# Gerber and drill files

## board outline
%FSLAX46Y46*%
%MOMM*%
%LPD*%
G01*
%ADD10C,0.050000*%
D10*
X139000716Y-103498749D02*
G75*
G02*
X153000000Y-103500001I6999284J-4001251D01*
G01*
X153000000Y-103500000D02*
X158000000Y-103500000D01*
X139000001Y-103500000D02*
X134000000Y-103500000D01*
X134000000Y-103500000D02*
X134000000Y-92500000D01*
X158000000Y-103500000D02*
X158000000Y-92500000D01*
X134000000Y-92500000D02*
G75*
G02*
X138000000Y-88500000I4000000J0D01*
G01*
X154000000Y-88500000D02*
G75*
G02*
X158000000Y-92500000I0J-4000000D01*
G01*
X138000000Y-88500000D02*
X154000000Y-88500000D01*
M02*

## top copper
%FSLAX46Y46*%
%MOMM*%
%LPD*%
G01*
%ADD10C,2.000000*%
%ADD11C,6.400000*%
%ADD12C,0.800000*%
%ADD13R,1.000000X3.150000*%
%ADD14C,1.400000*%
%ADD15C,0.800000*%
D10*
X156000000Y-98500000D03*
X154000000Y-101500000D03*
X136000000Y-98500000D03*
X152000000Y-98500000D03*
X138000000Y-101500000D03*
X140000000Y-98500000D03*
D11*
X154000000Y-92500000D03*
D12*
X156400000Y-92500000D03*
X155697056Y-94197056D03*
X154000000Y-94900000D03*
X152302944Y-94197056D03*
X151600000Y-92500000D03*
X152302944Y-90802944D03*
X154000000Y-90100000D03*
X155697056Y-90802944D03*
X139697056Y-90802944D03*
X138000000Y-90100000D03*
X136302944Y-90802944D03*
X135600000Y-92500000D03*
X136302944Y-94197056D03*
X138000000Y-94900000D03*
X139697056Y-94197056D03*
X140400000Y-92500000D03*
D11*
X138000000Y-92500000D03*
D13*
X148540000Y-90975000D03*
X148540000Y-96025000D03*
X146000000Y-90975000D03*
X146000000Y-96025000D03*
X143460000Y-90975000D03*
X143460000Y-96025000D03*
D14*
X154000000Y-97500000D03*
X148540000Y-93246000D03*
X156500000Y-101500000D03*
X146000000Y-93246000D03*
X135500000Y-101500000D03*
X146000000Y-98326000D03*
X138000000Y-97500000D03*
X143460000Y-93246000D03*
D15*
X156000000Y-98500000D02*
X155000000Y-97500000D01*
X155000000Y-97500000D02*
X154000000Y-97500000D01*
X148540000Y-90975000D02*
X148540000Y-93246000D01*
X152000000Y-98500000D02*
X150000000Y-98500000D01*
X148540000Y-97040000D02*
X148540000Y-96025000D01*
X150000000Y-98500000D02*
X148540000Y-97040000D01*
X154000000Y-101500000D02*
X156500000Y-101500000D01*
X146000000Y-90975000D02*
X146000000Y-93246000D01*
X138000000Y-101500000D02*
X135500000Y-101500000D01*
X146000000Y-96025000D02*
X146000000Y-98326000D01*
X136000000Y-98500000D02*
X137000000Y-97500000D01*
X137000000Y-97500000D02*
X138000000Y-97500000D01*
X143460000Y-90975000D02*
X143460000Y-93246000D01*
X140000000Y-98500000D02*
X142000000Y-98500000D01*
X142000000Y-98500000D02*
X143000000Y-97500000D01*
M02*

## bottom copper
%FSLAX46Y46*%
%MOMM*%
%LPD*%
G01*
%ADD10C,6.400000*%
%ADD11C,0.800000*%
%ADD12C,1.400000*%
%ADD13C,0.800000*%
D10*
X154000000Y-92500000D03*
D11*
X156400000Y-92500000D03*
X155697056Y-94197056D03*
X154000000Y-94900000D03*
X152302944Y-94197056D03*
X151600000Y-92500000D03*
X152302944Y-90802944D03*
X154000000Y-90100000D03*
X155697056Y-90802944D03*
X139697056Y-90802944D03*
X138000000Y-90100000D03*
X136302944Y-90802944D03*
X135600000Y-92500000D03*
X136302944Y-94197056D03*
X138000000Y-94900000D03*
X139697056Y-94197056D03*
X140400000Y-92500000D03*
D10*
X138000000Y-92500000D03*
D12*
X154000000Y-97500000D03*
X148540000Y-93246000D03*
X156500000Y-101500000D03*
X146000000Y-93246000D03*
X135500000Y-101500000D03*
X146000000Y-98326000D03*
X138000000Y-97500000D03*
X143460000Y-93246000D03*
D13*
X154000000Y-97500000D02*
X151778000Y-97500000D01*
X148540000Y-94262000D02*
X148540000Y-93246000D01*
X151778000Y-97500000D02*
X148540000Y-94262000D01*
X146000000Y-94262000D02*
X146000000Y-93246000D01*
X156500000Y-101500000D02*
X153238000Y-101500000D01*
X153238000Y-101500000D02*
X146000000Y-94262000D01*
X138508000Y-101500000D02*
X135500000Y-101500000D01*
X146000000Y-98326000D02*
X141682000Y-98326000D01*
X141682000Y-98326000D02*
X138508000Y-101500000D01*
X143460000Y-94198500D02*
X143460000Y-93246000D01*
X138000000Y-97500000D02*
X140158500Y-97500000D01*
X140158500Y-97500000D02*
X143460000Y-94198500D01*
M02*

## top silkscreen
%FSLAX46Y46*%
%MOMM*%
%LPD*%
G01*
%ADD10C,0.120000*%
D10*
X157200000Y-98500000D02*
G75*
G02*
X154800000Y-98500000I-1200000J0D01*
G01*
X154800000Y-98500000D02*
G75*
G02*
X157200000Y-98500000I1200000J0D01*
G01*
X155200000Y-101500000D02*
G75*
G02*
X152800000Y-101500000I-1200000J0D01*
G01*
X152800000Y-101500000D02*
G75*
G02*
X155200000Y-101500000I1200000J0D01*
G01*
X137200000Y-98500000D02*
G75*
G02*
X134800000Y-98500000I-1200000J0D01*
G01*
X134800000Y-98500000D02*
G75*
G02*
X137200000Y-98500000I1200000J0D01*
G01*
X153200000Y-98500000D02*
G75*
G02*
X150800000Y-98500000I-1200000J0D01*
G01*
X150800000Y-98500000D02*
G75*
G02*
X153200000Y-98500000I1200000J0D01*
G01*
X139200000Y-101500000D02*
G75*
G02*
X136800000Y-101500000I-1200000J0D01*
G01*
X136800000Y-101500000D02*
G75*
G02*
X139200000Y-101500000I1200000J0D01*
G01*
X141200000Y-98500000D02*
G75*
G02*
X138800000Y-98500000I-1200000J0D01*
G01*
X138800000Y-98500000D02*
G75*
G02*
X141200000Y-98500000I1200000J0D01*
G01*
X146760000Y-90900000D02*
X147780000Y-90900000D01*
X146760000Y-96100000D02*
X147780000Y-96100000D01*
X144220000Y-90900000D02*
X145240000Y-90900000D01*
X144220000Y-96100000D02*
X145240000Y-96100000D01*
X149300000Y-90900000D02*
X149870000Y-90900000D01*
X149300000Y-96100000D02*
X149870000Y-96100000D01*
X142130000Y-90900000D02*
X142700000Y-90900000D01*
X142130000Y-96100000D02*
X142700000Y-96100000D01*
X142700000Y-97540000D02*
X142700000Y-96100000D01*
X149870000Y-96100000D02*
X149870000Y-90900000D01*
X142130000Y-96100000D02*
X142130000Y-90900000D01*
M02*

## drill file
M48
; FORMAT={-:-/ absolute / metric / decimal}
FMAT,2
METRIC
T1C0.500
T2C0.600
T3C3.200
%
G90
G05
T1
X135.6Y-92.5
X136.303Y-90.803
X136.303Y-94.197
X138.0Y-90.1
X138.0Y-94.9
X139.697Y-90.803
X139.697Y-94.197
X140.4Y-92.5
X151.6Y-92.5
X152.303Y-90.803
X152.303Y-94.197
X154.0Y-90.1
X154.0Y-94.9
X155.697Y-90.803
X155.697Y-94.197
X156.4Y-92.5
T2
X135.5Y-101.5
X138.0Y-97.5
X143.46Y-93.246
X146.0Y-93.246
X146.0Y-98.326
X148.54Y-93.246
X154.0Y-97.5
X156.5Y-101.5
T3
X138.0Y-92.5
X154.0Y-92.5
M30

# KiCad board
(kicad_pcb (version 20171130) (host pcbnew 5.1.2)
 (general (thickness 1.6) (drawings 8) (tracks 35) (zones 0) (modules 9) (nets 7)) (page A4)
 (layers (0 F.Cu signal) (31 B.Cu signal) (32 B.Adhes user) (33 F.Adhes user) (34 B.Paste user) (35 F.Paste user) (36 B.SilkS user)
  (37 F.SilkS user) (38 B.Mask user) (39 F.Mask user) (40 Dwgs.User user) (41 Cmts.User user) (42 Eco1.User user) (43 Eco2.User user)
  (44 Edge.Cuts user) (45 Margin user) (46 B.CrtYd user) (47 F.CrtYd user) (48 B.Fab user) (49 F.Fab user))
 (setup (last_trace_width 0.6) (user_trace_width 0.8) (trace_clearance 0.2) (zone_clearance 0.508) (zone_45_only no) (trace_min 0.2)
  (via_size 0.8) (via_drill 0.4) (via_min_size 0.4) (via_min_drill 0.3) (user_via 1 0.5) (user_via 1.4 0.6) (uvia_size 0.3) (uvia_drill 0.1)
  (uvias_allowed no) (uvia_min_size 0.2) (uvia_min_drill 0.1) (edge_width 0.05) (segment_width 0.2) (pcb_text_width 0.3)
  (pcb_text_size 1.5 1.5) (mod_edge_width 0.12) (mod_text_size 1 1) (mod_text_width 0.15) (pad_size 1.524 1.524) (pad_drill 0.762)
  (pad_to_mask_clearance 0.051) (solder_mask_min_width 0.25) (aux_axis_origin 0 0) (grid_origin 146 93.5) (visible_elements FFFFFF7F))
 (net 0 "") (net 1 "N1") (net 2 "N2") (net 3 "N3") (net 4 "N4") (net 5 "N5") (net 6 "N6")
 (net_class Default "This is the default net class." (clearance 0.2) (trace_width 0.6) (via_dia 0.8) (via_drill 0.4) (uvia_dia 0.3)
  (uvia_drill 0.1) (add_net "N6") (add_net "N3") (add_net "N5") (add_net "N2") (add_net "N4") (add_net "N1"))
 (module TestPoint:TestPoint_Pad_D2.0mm (layer F.Cu) (at 156 98.5)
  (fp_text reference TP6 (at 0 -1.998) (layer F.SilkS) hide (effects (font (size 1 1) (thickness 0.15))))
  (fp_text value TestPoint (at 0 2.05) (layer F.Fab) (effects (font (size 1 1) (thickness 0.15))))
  (fp_circle (center 0 0) (end 0 1.2) (layer F.SilkS) (width 0.12))
  (pad 1 smd circle (at 0 0) (size 2 2) (layers F.Cu F.Mask) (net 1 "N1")))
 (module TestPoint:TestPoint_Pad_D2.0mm (layer F.Cu) (at 154 101.5)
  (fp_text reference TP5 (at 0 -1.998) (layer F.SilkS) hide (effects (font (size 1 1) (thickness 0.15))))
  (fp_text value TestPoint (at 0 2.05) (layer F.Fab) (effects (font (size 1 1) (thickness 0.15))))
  (fp_circle (center 0 0) (end 0 1.2) (layer F.SilkS) (width 0.12))
  (pad 1 smd circle (at 0 0) (size 2 2) (layers F.Cu F.Mask) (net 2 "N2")))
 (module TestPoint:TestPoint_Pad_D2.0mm (layer F.Cu) (at 136 98.5)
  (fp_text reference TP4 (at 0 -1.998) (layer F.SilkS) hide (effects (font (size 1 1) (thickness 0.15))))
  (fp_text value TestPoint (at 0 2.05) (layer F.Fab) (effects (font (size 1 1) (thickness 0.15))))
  (fp_circle (center 0 0) (end 0 1.2) (layer F.SilkS) (width 0.12))
  (pad 1 smd circle (at 0 0) (size 2 2) (layers F.Cu F.Mask) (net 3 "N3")))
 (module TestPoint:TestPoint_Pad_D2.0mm (layer F.Cu) (at 152 98.5)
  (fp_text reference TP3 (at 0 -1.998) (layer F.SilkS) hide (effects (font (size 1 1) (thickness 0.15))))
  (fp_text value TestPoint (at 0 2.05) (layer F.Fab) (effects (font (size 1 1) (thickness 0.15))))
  (fp_circle (center 0 0) (end 0 1.2) (layer F.SilkS) (width 0.12))
  (pad 1 smd circle (at 0 0) (size 2 2) (layers F.Cu F.Mask) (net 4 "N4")))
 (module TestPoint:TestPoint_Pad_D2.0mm (layer F.Cu) (at 138 101.5)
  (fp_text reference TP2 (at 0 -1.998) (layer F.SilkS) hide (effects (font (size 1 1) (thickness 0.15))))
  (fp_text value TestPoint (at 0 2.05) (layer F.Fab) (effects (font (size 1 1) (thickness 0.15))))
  (fp_circle (center 0 0) (end 0 1.2) (layer F.SilkS) (width 0.12))
  (pad 1 smd circle (at 0 0) (size 2 2) (layers F.Cu F.Mask) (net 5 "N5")))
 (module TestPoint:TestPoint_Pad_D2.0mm (layer F.Cu) (at 140 98.5)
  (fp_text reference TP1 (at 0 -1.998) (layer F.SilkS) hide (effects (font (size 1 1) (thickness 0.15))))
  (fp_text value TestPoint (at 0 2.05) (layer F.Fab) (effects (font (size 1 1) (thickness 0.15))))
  (fp_circle (center 0 0) (end 0 1.2) (layer F.SilkS) (width 0.12))
  (pad 1 smd circle (at 0 0) (size 2 2) (layers F.Cu F.Mask) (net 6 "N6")))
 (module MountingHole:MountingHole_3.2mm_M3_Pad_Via (layer F.Cu) (at 154 92.5)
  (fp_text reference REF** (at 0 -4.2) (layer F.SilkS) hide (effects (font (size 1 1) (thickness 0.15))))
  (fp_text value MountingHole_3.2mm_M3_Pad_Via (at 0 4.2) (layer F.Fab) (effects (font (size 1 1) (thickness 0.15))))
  (pad 1 thru_hole circle (at 0 0) (size 6.4 6.4) (drill 3.2) (layers *.Cu *.Mask))
  (pad 1 thru_hole circle (at 2.4 0) (size 0.8 0.8) (drill 0.5) (layers *.Cu *.Mask))
  (pad 1 thru_hole circle (at 1.697056 1.697056) (size 0.8 0.8) (drill 0.5) (layers *.Cu *.Mask))
  (pad 1 thru_hole circle (at 0 2.4) (size 0.8 0.8) (drill 0.5) (layers *.Cu *.Mask))
  (pad 1 thru_hole circle (at -1.697056 1.697056) (size 0.8 0.8) (drill 0.5) (layers *.Cu *.Mask))
  (pad 1 thru_hole circle (at -2.4 0) (size 0.8 0.8) (drill 0.5) (layers *.Cu *.Mask))
  (pad 1 thru_hole circle (at -1.697056 -1.697056) (size 0.8 0.8) (drill 0.5) (layers *.Cu *.Mask))
  (pad 1 thru_hole circle (at 0 -2.4) (size 0.8 0.8) (drill 0.5) (layers *.Cu *.Mask))
  (pad 1 thru_hole circle (at 1.697056 -1.697056) (size 0.8 0.8) (drill 0.5) (layers *.Cu *.Mask)))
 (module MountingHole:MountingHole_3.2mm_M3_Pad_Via (layer F.Cu) (at 138 92.5)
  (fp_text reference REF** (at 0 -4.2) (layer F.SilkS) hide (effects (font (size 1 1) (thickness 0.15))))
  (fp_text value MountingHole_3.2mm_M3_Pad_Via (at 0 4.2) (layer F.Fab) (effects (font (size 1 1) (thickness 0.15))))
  (pad 1 thru_hole circle (at 1.697056 -1.697056) (size 0.8 0.8) (drill 0.5) (layers *.Cu *.Mask))
  (pad 1 thru_hole circle (at 0 -2.4) (size 0.8 0.8) (drill 0.5) (layers *.Cu *.Mask))
  (pad 1 thru_hole circle (at -1.697056 -1.697056) (size 0.8 0.8) (drill 0.5) (layers *.Cu *.Mask))
  (pad 1 thru_hole circle (at -2.4 0) (size 0.8 0.8) (drill 0.5) (layers *.Cu *.Mask))
  (pad 1 thru_hole circle (at -1.697056 1.697056) (size 0.8 0.8) (drill 0.5) (layers *.Cu *.Mask))
  (pad 1 thru_hole circle (at 0 2.4) (size 0.8 0.8) (drill 0.5) (layers *.Cu *.Mask))
  (pad 1 thru_hole circle (at 1.697056 1.697056) (size 0.8 0.8) (drill 0.5) (layers *.Cu *.Mask))
  (pad 1 thru_hole circle (at 2.4 0) (size 0.8 0.8) (drill 0.5) (layers *.Cu *.Mask))
  (pad 1 thru_hole circle (at 0 0) (size 6.4 6.4) (drill 3.2) (layers *.Cu *.Mask)))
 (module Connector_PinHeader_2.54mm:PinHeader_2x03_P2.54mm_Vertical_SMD (layer F.Cu) (at 146 93.5 90)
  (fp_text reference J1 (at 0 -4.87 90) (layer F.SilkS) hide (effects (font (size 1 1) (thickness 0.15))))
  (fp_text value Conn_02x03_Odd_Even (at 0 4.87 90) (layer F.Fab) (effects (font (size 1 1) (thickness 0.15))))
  (fp_line (start 2.6 0.76) (end 2.6 1.78) (layer F.SilkS) (width 0.12))
  (fp_line (start -2.6 0.76) (end -2.6 1.78) (layer F.SilkS) (width 0.12))
  (fp_line (start 2.6 -1.78) (end 2.6 -0.76) (layer F.SilkS) (width 0.12))
  (fp_line (start -2.6 -1.78) (end -2.6 -0.76) (layer F.SilkS) (width 0.12))
  (fp_line (start 2.6 3.3) (end 2.6 3.87) (layer F.SilkS) (width 0.12))
  (fp_line (start -2.6 3.3) (end -2.6 3.87) (layer F.SilkS) (width 0.12))
  (fp_line (start 2.6 -3.87) (end 2.6 -3.3) (layer F.SilkS) (width 0.12))
  (fp_line (start -2.6 -3.87) (end -2.6 -3.3) (layer F.SilkS) (width 0.12))
  (fp_line (start -4.04 -3.3) (end -2.6 -3.3) (layer F.SilkS) (width 0.12))
  (fp_line (start -2.6 3.87) (end 2.6 3.87) (layer F.SilkS) (width 0.12))
  (fp_line (start -2.6 -3.87) (end 2.6 -3.87) (layer F.SilkS) (width 0.12))
  (pad 6 smd rect (at 2.525 2.54 90) (size 3.15 1) (layers F.Cu F.Paste F.Mask) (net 1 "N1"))
  (pad 5 smd rect (at -2.525 2.54 90) (size 3.15 1) (layers F.Cu F.Paste F.Mask) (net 4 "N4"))
  (pad 4 smd rect (at 2.525 0 90) (size 3.15 1) (layers F.Cu F.Paste F.Mask) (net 2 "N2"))
  (pad 3 smd rect (at -2.525 0 90) (size 3.15 1) (layers F.Cu F.Paste F.Mask) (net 5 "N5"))
  (pad 2 smd rect (at 2.525 -2.54 90) (size 3.15 1) (layers F.Cu F.Paste F.Mask) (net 3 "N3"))
  (pad 1 smd rect (at -2.525 -2.54 90) (size 3.15 1) (layers F.Cu F.Paste F.Mask) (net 6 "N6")))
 (gr_arc (start 146 107.5) (end 153 103.500001) (angle -120.5) (layer Edge.Cuts) (width 0.05))
 (gr_line (start 153 103.5) (end 158 103.5) (layer Edge.Cuts) (width 0.05))
 (gr_line (start 139.000001 103.5) (end 134 103.5) (layer Edge.Cuts) (width 0.05))
 (gr_line (start 134 103.5) (end 134 92.5) (layer Edge.Cuts) (width 0.05))
 (gr_line (start 158 103.5) (end 158 92.5) (layer Edge.Cuts) (width 0.05))
 (gr_arc (start 138 92.5) (end 138 88.5) (angle -90) (layer Edge.Cuts) (width 0.05))
 (gr_arc (start 154 92.5) (end 158 92.5) (angle -90) (layer Edge.Cuts) (width 0.05))
 (gr_line (start 138 88.5) (end 154 88.5) (layer Edge.Cuts) (width 0.05))
 (segment (start 156 98.5) (end 155 97.5) (width 0.8) (layer F.Cu) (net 1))
 (segment (start 155 97.5) (end 154 97.5) (width 0.8) (layer F.Cu) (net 1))
 (via (at 154 97.5) (size 1.4) (drill 0.6) (layers F.Cu B.Cu) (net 1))
 (via (at 148.54 93.246) (size 1.4) (drill 0.6) (layers F.Cu B.Cu) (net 1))
 (segment (start 148.54 90.975) (end 148.54 93.246) (width 0.8) (layer F.Cu) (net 1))
 (segment (start 154 97.5) (end 151.778 97.5) (width 0.8) (layer B.Cu) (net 1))
 (segment (start 148.54 94.262) (end 148.54 93.246) (width 0.8) (layer B.Cu) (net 1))
 (segment (start 151.778 97.5) (end 148.54 94.262) (width 0.8) (layer B.Cu) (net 1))
 (segment (start 152 98.5) (end 150 98.5) (width 0.8) (layer F.Cu) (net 4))
 (segment (start 148.54 97.04) (end 148.54 96.025) (width 0.8) (layer F.Cu) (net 4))
 (segment (start 150 98.5) (end 148.54 97.04) (width 0.8) (layer F.Cu) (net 4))
 (segment (start 154 101.5) (end 156.5 101.5) (width 0.8) (layer F.Cu) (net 2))
 (via (at 156.5 101.5) (size 1.4) (drill 0.6) (layers F.Cu B.Cu) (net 2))
 (via (at 146 93.246) (size 1.4) (drill 0.6) (layers F.Cu B.Cu) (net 2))
 (segment (start 146 90.975) (end 146 93.246) (width 0.8) (layer F.Cu) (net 2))
 (segment (start 146 94.262) (end 146 93.246) (width 0.8) (layer B.Cu) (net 2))
 (segment (start 156.5 101.5) (end 153.238 101.5) (width 0.8) (layer B.Cu) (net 2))
 (segment (start 153.238 101.5) (end 146 94.262) (width 0.8) (layer B.Cu) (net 2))
 (segment (start 138 101.5) (end 135.5 101.5) (width 0.8) (layer F.Cu) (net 5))
 (via (at 135.5 101.5) (size 1.4) (drill 0.6) (layers F.Cu B.Cu) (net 5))
 (via (at 146 98.326) (size 1.4) (drill 0.6) (layers F.Cu B.Cu) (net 5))
 (segment (start 146 96.025) (end 146 98.326) (width 0.8) (layer F.Cu) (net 5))
 (segment (start 138.508 101.5) (end 135.5 101.5) (width 0.8) (layer B.Cu) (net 5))
 (segment (start 146 98.326) (end 141.682 98.326) (width 0.8) (layer B.Cu) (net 5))
 (segment (start 141.682 98.326) (end 138.508 101.5) (width 0.8) (layer B.Cu) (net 5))
 (segment (start 136 98.5) (end 137 97.5) (width 0.8) (layer F.Cu) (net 3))
 (via (at 138 97.5) (size 1.4) (drill 0.6) (layers F.Cu B.Cu) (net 3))
 (segment (start 137 97.5) (end 138 97.5) (width 0.8) (layer F.Cu) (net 3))
 (via (at 143.46 93.246) (size 1.4) (drill 0.6) (layers F.Cu B.Cu) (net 3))
 (segment (start 143.46 90.975) (end 143.46 93.246) (width 0.8) (layer F.Cu) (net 3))
 (segment (start 143.46 94.1985) (end 143.46 93.246) (width 0.8) (layer B.Cu) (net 3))
 (segment (start 138 97.5) (end 140.1585 97.5) (width 0.8) (layer B.Cu) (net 3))
 (segment (start 140.1585 97.5) (end 143.46 94.1985) (width 0.8) (layer B.Cu) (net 3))
 (segment (start 140 98.5) (end 142 98.5) (width 0.8) (layer F.Cu) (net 6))
 (segment (start 142 98.5) (end 143 97.5) (width 0.8) (layer F.Cu) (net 6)))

